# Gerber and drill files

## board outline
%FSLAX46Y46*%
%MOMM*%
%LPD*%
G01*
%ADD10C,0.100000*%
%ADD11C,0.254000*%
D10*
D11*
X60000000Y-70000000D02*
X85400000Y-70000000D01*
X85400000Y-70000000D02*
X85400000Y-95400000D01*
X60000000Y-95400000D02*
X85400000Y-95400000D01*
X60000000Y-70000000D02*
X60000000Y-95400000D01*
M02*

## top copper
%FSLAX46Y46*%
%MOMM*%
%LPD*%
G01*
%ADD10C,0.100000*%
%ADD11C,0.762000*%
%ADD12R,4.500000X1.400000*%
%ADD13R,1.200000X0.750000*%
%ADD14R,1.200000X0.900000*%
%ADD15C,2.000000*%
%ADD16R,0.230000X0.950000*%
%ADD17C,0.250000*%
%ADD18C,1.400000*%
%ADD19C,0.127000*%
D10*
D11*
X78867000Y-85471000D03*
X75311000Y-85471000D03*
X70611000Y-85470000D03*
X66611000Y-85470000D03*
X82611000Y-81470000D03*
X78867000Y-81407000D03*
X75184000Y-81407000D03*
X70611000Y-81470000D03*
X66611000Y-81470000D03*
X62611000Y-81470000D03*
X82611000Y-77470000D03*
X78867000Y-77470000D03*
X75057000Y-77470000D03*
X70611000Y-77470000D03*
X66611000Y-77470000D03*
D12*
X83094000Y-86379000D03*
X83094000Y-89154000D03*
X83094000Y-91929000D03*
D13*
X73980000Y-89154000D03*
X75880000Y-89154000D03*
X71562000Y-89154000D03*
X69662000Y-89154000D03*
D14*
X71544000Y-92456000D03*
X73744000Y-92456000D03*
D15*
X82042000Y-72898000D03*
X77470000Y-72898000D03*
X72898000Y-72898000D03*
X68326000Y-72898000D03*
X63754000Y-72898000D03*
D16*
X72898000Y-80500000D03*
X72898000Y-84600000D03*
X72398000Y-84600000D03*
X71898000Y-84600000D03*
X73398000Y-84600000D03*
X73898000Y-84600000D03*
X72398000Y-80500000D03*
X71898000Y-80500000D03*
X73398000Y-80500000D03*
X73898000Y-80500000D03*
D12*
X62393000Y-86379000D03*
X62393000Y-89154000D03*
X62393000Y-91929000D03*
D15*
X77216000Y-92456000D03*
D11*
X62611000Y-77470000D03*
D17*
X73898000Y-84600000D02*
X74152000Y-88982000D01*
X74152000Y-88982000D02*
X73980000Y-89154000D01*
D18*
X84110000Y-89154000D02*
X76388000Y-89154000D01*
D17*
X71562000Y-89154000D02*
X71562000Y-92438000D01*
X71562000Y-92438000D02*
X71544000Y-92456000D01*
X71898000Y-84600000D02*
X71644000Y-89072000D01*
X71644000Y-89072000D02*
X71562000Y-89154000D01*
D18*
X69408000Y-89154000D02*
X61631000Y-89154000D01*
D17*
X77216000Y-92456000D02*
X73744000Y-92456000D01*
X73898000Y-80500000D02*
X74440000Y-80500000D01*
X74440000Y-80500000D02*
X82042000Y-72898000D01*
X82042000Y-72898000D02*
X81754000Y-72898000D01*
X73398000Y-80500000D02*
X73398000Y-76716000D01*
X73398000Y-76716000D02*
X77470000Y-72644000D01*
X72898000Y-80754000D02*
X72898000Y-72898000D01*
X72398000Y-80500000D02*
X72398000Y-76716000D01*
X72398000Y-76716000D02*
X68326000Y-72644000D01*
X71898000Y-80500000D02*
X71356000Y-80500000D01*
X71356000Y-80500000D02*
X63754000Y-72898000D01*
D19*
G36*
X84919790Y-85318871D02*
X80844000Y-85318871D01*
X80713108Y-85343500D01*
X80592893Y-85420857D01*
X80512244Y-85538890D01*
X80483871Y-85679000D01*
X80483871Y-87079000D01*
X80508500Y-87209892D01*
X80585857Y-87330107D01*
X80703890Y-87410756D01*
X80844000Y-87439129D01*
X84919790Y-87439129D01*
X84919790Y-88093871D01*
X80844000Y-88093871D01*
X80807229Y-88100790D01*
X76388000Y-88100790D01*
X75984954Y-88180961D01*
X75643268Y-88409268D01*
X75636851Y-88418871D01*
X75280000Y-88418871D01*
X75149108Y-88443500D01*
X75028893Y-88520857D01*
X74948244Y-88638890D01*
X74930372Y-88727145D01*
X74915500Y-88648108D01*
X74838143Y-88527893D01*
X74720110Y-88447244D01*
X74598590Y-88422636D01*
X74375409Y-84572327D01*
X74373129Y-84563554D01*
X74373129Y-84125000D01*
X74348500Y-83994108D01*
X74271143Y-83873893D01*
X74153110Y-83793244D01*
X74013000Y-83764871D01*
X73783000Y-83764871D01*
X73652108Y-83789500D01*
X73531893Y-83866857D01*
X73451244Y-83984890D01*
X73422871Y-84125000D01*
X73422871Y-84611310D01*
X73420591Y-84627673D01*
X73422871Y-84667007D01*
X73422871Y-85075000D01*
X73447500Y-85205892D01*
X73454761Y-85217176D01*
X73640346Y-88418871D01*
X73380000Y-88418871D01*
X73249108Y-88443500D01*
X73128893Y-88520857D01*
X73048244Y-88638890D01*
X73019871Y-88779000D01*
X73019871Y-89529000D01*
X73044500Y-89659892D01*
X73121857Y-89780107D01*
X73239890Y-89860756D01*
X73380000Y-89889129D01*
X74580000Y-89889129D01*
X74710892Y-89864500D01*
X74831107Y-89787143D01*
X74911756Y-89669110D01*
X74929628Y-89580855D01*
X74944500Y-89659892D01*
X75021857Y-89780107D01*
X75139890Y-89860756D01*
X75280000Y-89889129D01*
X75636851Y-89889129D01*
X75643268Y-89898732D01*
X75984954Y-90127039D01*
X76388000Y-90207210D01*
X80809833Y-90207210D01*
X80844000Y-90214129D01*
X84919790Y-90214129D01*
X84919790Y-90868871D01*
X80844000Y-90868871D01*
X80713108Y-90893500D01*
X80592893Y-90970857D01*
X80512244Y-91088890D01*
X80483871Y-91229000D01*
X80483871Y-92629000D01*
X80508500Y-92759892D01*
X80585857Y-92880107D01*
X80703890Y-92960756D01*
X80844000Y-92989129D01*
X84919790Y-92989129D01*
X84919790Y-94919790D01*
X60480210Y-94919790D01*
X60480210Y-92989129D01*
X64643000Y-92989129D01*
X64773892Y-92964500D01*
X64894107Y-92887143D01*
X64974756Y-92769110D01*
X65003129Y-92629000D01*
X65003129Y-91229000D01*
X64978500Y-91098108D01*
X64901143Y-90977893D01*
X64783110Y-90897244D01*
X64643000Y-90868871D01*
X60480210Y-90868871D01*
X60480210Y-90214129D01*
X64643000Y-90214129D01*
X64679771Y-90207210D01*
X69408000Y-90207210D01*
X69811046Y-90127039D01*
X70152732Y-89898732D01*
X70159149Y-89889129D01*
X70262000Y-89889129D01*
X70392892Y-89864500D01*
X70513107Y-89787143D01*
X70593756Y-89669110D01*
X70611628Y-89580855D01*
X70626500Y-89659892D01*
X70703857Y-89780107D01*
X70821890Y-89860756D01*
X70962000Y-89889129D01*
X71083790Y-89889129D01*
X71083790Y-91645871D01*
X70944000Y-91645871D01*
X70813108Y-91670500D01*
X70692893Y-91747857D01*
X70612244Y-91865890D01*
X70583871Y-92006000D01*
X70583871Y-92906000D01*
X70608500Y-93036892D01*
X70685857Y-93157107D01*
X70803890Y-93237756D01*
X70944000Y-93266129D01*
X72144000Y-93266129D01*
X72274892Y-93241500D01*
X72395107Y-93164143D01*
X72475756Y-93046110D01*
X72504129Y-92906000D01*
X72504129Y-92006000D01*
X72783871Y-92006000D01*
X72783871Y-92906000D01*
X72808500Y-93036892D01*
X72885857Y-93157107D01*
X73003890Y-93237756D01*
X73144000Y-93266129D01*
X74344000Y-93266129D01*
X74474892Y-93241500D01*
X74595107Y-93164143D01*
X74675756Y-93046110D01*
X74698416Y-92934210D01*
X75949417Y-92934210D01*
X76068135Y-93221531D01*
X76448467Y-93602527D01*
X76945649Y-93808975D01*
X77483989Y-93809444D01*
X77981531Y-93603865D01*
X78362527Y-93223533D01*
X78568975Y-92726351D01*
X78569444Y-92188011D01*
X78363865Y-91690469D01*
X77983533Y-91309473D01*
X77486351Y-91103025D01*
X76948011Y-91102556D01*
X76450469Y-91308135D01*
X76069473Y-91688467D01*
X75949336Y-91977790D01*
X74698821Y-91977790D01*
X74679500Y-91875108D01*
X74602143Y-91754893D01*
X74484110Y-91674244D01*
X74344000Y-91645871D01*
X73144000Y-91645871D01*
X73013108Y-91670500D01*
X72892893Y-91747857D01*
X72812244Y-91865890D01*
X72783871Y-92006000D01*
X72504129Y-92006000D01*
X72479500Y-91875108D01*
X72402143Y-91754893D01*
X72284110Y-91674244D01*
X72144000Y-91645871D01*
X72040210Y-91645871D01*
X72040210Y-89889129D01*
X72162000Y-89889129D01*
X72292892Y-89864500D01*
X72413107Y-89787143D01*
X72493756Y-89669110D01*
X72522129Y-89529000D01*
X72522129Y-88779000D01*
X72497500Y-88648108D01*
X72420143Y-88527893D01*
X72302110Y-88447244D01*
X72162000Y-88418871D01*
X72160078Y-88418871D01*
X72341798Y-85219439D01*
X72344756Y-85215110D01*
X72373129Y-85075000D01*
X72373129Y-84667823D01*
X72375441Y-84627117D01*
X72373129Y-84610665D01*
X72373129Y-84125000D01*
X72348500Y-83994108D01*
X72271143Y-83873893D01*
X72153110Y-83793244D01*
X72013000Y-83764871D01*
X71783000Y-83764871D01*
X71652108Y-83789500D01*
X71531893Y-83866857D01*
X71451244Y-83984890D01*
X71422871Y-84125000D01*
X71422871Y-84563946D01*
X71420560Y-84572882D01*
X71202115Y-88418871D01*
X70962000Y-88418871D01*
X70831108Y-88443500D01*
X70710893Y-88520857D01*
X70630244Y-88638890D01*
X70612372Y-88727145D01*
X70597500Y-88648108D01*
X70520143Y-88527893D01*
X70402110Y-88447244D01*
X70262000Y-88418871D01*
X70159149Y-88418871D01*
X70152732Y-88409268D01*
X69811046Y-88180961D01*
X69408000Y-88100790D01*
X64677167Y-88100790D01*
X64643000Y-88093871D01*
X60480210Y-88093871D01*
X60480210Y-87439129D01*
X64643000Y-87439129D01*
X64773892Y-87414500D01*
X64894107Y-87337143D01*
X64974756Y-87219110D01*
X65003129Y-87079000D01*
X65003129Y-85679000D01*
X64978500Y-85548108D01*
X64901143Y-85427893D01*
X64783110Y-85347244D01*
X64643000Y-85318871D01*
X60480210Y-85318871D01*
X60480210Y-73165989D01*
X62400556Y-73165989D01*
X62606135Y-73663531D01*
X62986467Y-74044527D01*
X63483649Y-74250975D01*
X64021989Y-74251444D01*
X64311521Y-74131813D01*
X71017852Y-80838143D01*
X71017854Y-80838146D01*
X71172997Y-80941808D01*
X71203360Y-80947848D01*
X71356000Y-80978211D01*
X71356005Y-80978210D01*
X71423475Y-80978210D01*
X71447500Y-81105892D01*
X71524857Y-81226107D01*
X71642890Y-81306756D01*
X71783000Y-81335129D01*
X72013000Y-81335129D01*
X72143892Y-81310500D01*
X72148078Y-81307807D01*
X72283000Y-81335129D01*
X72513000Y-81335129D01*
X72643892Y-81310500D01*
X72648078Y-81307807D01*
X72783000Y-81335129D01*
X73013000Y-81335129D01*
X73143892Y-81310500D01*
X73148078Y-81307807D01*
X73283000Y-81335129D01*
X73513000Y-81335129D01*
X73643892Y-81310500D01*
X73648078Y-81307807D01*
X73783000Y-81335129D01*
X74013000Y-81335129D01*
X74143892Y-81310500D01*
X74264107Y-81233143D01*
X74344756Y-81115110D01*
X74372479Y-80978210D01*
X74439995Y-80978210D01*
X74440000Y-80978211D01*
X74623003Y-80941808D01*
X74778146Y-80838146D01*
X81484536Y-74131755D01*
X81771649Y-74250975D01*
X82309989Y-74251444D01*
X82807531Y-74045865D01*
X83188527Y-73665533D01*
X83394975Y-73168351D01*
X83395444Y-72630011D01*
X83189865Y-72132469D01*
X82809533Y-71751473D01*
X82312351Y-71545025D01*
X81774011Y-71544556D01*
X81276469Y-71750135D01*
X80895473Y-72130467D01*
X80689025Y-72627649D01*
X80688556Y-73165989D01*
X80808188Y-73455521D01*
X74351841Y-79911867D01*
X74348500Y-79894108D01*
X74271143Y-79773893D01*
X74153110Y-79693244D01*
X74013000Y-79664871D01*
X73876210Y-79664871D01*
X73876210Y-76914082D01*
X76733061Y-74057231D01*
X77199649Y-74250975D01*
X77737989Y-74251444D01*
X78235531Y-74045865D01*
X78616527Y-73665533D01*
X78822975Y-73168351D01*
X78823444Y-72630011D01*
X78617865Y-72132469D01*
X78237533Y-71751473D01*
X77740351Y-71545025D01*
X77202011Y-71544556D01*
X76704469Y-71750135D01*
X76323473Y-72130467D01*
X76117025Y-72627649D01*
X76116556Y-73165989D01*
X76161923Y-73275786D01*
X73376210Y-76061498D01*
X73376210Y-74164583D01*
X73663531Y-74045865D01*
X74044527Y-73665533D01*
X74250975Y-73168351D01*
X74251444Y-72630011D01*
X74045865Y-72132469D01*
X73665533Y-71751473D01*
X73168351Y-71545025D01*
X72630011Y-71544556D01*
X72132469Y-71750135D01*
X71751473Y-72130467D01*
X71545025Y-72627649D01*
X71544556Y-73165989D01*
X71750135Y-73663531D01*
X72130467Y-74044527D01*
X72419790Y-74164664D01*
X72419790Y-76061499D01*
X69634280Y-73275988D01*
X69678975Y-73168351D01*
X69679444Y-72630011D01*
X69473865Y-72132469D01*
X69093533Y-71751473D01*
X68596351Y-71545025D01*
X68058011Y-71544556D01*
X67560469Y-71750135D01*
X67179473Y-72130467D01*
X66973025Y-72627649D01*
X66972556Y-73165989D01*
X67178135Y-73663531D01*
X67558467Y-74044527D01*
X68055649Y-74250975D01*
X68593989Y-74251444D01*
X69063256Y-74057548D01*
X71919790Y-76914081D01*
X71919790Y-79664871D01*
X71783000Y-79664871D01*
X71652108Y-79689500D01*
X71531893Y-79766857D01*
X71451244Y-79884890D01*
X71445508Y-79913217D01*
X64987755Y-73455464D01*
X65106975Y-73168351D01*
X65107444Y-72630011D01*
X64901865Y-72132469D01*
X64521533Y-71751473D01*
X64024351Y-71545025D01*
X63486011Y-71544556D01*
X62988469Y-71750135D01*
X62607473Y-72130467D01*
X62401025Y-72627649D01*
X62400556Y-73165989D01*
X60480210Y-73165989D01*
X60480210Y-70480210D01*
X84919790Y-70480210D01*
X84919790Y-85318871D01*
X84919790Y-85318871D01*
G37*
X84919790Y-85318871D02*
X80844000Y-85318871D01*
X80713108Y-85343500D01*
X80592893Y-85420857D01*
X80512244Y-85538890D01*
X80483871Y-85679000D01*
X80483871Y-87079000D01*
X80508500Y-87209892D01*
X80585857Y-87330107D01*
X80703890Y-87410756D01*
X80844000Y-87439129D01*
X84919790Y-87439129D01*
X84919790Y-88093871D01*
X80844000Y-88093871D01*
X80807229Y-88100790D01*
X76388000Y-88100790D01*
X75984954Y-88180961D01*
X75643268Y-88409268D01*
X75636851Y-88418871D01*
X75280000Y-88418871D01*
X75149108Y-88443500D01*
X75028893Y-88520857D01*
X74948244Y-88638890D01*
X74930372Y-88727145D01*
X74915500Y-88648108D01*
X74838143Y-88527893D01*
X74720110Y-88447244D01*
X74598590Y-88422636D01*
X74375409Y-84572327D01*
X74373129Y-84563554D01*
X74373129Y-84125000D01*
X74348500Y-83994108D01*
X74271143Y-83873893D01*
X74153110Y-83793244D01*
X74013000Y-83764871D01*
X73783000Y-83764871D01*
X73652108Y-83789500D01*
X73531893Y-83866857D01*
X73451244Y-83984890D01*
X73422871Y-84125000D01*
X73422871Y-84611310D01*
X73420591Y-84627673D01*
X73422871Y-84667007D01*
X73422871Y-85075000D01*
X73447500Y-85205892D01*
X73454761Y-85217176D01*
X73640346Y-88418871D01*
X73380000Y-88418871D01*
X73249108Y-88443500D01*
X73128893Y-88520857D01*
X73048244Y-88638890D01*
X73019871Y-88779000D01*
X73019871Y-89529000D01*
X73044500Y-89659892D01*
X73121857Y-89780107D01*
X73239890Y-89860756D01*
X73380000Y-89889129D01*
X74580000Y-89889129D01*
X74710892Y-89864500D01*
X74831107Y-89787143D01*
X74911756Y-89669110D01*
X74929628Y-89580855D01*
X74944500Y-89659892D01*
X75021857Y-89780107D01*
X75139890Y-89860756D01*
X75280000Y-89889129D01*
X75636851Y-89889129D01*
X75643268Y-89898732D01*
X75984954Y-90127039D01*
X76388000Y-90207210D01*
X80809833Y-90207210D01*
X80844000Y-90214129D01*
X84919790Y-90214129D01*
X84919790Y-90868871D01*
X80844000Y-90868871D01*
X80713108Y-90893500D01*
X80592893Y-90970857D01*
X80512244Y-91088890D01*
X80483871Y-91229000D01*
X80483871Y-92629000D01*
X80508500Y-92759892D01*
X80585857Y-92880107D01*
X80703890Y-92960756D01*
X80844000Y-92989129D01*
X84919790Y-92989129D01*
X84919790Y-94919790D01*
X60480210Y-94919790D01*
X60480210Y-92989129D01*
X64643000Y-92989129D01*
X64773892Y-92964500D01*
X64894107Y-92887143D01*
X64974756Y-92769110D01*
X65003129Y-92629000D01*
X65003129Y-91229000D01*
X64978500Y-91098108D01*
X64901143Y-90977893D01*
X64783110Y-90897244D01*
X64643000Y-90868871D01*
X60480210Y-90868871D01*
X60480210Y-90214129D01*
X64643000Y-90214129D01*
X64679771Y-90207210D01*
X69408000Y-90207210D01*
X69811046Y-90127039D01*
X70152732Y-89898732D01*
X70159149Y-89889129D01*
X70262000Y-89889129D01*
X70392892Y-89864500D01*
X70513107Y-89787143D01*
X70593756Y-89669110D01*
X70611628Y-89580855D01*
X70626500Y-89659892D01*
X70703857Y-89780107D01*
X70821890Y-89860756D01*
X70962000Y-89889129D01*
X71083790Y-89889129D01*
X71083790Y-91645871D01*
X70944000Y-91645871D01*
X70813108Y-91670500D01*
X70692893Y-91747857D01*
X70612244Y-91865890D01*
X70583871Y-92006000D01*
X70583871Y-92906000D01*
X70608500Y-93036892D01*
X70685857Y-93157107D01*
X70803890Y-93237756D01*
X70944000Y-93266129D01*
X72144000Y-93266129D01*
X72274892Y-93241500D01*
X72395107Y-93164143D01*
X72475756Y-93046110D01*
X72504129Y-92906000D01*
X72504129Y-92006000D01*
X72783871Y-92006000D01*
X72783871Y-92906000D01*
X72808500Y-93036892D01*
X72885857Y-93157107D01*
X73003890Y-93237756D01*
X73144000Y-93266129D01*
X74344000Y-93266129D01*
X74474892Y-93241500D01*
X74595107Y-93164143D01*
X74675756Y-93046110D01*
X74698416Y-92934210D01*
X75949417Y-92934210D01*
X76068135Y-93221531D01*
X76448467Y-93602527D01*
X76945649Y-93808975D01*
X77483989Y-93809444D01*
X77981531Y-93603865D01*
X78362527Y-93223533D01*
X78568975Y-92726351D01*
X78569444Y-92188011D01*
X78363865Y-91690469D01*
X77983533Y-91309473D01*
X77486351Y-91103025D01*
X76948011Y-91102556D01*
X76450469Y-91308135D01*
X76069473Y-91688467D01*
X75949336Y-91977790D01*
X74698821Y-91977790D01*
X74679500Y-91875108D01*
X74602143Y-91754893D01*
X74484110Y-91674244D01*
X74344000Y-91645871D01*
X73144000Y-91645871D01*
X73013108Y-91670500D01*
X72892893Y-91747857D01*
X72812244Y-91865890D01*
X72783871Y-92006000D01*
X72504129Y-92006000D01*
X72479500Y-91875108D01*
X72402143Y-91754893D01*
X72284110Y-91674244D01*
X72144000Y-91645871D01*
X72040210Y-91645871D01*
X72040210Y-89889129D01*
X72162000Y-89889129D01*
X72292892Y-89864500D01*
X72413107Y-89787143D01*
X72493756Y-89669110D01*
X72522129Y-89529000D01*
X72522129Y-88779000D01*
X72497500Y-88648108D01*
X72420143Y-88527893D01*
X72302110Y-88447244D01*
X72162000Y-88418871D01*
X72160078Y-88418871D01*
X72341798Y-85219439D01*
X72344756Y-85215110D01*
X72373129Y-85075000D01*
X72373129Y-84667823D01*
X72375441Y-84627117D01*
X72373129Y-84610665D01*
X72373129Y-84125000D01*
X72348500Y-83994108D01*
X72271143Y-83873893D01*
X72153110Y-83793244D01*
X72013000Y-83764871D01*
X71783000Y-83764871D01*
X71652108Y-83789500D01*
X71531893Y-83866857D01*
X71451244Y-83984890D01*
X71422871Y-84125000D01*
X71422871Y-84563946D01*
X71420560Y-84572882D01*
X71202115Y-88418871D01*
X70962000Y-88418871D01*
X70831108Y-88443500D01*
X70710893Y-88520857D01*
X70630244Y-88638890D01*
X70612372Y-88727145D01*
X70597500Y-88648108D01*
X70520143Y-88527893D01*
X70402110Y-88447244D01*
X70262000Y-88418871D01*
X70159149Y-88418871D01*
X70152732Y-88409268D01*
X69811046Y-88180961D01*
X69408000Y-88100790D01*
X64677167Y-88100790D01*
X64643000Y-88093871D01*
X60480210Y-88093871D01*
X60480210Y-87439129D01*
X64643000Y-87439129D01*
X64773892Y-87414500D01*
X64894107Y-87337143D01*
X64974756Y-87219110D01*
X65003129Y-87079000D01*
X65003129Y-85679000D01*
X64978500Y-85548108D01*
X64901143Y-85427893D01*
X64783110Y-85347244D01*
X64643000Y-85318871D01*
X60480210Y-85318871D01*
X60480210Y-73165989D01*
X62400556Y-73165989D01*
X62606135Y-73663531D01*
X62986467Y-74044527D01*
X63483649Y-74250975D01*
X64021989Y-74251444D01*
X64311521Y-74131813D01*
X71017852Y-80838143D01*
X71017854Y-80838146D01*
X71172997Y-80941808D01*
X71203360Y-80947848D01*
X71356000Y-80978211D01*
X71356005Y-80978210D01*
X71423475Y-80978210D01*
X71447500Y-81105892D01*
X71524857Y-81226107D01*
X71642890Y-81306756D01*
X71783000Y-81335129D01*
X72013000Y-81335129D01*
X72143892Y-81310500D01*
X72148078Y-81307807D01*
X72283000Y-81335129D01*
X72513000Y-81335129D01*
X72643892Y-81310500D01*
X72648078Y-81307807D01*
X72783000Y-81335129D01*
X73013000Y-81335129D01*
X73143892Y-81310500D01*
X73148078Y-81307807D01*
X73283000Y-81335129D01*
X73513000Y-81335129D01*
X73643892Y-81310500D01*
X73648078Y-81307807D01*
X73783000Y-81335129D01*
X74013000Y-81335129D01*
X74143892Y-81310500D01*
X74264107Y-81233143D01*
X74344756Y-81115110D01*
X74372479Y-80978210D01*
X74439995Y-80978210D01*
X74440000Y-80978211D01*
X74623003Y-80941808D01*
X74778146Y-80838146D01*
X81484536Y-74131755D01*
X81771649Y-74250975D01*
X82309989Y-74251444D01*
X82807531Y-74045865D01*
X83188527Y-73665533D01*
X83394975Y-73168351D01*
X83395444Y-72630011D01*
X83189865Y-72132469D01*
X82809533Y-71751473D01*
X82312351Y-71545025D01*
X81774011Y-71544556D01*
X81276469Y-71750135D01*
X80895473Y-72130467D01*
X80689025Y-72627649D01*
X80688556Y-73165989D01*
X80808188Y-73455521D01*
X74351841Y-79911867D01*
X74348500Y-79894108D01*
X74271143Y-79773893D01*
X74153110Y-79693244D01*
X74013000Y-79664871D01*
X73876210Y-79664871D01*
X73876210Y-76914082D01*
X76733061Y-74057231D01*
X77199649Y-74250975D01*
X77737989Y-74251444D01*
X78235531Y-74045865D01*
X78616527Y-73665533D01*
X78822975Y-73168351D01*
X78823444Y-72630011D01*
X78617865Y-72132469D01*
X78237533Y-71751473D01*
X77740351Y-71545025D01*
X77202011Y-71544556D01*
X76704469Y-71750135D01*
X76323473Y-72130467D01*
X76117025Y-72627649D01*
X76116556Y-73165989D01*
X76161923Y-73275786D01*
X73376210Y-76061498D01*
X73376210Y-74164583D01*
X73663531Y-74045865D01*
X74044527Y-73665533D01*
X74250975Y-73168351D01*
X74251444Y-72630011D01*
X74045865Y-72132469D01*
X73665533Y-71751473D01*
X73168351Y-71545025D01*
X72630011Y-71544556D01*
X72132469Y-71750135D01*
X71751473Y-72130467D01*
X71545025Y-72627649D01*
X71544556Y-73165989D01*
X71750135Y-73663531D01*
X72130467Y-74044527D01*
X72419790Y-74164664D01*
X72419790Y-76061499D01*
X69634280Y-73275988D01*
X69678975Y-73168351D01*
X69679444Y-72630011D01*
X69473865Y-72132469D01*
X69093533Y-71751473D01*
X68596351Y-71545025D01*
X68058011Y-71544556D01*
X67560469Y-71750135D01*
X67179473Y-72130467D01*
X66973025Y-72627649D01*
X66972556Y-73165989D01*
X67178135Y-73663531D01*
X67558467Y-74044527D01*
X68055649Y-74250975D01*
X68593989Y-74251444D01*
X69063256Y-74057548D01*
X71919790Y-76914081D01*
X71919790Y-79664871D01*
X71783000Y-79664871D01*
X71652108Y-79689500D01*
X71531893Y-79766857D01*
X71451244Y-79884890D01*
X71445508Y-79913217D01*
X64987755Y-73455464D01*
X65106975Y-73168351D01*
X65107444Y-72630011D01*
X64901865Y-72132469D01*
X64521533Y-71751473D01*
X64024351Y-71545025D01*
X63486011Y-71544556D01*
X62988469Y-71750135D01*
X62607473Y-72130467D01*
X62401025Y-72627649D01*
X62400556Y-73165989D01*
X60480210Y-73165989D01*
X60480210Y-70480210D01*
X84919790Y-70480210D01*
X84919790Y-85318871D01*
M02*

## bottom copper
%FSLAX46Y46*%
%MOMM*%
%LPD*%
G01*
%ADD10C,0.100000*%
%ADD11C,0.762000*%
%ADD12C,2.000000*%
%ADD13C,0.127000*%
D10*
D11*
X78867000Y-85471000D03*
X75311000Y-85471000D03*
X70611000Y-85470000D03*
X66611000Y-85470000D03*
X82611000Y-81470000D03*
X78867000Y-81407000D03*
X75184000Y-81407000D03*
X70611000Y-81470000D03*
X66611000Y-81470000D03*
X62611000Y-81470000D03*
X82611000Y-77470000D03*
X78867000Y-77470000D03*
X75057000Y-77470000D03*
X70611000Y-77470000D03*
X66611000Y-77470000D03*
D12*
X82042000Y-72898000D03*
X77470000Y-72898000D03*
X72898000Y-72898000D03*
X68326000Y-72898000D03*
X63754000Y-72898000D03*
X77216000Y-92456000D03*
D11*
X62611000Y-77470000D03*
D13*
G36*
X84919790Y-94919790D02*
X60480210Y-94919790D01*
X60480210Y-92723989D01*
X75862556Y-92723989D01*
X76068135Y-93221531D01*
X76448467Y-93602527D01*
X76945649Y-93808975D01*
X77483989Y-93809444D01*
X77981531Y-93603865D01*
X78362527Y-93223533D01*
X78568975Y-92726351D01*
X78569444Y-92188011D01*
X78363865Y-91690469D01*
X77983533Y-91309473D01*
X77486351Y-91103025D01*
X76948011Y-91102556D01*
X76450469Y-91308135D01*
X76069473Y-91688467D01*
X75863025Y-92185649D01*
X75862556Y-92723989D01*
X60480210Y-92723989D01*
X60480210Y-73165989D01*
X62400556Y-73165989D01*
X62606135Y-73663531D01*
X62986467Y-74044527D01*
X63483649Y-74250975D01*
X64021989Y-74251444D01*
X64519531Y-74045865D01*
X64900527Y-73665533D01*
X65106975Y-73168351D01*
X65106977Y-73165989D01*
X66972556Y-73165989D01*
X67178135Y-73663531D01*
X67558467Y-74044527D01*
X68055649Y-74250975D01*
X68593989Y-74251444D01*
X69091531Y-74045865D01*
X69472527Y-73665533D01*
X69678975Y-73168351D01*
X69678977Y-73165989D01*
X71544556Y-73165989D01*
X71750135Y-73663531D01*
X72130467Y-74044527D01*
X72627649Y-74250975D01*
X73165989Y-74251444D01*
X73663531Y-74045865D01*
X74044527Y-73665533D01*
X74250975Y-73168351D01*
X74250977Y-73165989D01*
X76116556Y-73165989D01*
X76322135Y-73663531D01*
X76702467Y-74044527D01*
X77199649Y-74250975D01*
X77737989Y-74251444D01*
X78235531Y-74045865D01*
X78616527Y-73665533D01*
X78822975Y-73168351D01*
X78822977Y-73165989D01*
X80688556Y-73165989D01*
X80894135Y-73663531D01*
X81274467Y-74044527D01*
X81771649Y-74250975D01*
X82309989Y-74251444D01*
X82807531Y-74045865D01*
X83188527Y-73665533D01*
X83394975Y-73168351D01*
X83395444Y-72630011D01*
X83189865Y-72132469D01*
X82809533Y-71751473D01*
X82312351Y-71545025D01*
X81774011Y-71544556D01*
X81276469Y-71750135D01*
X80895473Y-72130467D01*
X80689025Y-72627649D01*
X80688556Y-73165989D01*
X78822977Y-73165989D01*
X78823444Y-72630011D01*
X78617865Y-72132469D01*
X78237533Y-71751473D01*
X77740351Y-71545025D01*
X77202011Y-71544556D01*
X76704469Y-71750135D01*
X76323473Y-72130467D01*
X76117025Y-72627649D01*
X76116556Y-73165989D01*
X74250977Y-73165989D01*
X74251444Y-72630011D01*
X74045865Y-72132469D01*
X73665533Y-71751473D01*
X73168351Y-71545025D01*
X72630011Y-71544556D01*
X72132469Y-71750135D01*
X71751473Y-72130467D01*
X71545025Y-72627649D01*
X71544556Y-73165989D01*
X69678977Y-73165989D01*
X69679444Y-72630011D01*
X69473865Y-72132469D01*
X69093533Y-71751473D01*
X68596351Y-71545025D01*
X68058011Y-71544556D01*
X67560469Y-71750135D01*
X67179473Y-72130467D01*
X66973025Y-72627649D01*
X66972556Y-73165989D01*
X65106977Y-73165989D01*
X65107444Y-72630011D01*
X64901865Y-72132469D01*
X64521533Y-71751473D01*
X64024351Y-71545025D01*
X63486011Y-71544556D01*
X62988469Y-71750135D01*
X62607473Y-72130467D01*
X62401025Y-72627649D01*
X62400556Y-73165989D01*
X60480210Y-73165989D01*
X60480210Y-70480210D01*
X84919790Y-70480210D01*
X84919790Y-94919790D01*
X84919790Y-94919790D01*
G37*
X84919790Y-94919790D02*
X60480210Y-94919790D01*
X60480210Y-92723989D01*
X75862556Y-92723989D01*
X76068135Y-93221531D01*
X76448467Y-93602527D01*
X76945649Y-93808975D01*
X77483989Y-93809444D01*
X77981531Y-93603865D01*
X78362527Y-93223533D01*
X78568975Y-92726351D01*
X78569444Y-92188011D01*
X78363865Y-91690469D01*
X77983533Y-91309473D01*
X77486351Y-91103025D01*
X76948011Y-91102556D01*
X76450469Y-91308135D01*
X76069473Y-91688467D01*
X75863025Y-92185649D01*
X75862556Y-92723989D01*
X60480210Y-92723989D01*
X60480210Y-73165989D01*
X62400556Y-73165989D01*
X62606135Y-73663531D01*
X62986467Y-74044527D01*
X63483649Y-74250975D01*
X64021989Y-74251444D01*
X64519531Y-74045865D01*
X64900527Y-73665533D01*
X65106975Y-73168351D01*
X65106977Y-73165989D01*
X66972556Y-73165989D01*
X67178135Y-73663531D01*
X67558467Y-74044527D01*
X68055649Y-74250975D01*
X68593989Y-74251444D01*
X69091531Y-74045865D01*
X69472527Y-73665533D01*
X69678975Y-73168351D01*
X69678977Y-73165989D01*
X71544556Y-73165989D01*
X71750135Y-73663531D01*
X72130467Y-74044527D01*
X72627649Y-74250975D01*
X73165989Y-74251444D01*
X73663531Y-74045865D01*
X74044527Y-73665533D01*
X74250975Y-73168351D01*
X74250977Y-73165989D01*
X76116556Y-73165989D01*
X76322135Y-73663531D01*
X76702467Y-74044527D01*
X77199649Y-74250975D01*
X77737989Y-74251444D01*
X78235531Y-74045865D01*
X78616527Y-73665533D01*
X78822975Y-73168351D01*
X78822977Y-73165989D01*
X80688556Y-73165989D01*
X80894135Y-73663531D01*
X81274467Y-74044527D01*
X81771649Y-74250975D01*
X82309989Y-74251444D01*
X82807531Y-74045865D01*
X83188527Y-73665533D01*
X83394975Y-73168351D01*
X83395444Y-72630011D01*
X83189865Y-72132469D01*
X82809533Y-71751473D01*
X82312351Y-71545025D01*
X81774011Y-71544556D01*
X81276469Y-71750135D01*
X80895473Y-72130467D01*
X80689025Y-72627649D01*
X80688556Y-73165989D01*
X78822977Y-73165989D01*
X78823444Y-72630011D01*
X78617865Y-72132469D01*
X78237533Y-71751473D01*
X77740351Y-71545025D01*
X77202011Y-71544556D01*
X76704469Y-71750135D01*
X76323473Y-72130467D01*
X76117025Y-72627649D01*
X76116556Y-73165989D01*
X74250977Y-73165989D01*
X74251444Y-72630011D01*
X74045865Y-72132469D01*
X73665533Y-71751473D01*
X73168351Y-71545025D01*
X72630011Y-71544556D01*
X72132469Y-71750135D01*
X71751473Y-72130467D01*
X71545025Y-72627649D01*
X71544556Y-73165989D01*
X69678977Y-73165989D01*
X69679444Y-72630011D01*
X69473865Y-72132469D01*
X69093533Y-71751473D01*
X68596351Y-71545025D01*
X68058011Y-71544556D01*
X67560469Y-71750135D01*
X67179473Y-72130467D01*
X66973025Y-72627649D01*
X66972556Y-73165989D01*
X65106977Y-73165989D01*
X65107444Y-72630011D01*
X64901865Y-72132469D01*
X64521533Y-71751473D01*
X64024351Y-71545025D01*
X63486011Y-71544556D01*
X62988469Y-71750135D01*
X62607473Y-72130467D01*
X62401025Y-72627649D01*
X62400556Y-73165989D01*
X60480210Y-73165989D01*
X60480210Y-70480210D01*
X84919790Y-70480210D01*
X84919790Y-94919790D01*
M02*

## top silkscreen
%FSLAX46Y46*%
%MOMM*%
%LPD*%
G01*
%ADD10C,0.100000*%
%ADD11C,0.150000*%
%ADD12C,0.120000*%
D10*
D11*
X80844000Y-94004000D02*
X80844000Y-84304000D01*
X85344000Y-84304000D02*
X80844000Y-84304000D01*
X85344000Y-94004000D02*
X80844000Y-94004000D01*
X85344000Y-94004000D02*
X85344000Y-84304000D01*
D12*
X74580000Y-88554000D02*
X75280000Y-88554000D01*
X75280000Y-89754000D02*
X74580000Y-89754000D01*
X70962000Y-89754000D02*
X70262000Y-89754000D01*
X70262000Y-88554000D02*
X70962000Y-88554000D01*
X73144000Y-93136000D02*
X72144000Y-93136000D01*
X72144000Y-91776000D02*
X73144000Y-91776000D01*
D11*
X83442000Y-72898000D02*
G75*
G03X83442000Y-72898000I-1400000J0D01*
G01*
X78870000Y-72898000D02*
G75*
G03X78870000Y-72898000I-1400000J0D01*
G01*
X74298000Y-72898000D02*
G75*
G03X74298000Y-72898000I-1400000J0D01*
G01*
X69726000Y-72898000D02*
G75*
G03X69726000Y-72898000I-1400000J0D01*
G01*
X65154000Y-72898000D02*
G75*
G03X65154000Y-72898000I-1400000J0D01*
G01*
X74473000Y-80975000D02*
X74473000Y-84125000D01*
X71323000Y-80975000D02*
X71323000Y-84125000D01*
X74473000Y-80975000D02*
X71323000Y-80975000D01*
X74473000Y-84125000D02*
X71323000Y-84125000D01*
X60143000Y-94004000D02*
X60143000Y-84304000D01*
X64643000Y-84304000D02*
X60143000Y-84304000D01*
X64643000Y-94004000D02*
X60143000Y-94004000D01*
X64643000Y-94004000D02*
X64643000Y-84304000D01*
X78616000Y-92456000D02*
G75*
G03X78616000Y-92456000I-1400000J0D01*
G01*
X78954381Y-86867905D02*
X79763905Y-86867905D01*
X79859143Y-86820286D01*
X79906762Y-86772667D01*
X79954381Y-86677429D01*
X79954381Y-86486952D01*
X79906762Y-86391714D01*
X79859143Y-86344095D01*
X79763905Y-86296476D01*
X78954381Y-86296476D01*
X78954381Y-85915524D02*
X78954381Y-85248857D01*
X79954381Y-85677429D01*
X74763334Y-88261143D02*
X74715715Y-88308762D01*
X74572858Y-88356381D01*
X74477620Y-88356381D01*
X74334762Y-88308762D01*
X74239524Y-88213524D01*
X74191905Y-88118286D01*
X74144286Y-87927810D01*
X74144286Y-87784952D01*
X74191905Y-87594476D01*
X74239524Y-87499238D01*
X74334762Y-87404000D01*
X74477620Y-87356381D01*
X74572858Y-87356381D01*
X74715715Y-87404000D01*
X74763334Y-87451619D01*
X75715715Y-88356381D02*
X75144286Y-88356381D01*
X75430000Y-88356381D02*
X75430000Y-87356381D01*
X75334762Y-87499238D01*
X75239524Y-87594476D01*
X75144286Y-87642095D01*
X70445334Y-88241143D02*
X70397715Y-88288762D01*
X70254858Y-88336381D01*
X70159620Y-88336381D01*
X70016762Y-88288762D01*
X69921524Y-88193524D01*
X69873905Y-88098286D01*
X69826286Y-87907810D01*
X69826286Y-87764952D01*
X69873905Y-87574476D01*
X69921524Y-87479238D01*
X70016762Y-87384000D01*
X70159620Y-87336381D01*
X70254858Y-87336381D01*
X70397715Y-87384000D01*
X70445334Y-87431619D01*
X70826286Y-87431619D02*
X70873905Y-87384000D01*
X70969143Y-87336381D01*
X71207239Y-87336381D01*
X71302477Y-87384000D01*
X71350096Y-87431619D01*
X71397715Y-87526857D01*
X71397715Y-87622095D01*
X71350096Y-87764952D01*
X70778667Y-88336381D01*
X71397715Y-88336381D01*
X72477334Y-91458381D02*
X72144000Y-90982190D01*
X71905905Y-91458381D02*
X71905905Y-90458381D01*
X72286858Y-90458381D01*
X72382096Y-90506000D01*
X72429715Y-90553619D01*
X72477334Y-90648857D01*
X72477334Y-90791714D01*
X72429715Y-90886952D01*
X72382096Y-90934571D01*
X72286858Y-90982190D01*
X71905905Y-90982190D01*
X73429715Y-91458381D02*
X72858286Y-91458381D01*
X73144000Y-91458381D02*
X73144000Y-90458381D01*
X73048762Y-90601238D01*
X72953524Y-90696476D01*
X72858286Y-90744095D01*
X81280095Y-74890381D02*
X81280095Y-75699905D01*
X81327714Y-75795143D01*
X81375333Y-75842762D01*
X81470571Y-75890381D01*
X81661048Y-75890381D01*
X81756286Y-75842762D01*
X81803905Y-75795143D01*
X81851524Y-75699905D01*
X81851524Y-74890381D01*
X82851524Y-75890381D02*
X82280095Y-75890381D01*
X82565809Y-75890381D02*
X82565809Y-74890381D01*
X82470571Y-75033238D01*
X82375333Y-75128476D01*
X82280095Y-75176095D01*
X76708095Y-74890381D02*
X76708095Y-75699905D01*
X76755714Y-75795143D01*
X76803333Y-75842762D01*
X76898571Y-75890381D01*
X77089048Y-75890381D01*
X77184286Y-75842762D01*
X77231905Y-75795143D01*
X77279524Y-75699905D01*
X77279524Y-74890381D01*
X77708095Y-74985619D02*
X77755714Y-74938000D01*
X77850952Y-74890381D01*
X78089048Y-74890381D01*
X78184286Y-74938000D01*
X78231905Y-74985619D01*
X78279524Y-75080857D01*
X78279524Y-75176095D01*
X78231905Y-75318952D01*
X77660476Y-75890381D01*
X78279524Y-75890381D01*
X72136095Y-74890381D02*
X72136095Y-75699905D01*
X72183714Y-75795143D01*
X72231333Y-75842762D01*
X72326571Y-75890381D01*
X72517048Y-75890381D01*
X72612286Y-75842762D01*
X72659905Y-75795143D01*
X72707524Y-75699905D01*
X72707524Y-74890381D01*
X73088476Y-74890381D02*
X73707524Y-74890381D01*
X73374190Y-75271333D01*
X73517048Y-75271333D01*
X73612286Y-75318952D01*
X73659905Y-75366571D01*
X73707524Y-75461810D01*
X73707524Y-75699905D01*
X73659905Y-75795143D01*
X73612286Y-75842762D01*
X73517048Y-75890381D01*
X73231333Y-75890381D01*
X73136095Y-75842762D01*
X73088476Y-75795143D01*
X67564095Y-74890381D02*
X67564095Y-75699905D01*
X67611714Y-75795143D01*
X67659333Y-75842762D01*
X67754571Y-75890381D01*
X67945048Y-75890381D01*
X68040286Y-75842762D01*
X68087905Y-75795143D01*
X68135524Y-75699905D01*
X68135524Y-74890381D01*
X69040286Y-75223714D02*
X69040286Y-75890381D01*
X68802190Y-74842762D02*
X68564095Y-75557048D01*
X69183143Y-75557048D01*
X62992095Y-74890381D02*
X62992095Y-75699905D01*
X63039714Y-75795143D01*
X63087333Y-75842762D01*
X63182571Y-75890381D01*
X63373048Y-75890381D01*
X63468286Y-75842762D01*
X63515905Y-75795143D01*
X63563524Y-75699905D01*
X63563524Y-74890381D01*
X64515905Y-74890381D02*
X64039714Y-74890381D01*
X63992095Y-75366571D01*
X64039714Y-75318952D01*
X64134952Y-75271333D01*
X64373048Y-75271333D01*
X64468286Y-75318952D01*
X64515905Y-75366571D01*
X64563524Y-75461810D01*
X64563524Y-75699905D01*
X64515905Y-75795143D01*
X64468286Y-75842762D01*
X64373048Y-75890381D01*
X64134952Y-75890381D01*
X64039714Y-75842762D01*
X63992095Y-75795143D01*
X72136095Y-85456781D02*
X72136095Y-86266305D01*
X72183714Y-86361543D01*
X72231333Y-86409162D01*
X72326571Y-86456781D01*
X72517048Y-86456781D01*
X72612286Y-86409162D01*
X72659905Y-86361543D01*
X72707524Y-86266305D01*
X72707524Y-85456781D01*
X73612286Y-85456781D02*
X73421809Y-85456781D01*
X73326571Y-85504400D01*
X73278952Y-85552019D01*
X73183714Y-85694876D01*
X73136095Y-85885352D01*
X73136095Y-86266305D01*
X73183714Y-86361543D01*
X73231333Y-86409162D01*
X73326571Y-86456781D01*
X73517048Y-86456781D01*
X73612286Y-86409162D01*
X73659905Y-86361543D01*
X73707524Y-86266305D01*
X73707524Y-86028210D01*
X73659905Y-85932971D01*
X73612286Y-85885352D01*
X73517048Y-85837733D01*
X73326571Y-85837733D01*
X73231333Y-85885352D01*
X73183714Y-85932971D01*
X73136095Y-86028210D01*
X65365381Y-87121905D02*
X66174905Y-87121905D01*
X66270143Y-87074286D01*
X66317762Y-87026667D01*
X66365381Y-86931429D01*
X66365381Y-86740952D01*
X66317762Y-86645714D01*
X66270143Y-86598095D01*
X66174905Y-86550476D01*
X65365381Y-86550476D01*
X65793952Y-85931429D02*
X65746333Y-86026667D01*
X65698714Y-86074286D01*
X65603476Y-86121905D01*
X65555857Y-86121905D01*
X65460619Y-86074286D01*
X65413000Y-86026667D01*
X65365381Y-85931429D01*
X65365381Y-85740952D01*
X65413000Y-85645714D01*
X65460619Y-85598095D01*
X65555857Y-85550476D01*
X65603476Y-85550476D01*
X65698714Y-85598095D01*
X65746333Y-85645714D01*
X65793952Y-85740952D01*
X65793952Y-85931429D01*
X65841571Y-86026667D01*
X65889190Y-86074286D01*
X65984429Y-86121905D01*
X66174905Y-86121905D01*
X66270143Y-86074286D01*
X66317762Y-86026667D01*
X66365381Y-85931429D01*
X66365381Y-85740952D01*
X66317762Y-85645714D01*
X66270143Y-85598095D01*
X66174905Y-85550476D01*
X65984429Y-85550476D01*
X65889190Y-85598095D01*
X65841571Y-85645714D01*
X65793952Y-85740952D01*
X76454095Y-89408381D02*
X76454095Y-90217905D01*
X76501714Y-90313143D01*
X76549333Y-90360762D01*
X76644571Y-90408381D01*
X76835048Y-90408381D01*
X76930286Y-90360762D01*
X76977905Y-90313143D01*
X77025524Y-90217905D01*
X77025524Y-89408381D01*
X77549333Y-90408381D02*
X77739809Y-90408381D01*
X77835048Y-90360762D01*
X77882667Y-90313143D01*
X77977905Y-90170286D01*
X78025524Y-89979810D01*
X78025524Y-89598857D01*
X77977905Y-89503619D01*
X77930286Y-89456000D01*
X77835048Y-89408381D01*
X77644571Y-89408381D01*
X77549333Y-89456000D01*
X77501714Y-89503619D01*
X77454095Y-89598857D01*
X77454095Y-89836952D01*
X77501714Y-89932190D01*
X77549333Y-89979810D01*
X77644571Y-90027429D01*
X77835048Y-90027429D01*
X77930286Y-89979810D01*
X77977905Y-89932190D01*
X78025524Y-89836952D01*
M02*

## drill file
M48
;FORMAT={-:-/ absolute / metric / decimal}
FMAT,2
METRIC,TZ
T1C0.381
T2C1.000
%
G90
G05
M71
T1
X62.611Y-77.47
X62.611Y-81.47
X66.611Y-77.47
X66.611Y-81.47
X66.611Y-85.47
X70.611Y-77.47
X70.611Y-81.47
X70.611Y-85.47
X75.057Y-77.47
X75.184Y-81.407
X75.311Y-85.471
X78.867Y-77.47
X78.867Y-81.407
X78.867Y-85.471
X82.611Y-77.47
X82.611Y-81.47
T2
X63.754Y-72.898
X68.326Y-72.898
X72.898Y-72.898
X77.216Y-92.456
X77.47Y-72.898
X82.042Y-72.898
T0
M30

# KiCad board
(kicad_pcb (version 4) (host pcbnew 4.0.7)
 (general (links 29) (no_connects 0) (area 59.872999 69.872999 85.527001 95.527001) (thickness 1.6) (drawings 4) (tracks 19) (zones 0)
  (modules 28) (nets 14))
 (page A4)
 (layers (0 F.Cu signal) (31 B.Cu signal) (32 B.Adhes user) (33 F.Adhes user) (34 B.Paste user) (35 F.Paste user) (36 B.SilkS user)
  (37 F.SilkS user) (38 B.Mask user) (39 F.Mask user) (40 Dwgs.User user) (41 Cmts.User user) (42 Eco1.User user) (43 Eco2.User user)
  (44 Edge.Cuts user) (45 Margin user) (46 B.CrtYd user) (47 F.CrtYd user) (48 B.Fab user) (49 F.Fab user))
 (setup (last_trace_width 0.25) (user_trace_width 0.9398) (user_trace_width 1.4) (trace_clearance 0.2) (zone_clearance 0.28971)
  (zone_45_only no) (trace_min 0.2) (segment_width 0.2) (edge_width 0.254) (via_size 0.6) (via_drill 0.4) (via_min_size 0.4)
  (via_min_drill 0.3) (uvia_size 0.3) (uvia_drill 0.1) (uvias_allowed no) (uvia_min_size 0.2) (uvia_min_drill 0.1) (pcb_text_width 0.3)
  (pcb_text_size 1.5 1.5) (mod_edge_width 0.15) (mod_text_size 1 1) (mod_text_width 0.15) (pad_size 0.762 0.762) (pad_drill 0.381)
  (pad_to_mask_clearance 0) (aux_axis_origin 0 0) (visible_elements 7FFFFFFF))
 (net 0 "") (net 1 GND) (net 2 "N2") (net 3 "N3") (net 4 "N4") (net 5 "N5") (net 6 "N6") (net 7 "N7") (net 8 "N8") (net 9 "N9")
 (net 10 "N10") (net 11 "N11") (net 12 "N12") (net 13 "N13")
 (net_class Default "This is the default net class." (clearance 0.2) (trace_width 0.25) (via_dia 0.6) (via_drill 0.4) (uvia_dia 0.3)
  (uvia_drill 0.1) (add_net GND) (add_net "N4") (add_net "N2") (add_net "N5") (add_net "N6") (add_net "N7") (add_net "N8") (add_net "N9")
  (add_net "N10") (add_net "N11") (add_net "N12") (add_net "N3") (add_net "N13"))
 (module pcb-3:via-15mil (layer B.Cu) (at 78.867 85.471)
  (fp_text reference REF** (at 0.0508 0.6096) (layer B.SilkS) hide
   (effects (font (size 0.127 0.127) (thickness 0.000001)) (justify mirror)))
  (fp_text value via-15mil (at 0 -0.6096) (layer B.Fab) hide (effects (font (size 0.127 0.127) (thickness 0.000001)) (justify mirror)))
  (pad 1 thru_hole circle (at 0 0) (size 0.762 0.762) (drill 0.381) (layers *.Cu) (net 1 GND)))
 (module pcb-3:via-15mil (layer F.Cu) (at 75.311 85.471)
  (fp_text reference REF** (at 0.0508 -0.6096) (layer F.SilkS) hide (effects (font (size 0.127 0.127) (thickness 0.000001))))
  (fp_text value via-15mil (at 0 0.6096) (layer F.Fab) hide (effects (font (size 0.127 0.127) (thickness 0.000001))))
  (pad 1 thru_hole circle (at 0 0) (size 0.762 0.762) (drill 0.381) (layers *.Cu) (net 1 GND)))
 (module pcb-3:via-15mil (layer F.Cu) (at 70.611 85.47)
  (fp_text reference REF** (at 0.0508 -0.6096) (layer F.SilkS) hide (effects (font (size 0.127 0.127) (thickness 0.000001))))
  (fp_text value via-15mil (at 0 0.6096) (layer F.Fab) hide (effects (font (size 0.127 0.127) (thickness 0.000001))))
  (pad 1 thru_hole circle (at 0 0) (size 0.762 0.762) (drill 0.381) (layers *.Cu) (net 1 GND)))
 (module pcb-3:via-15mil (layer F.Cu) (at 66.611 85.47)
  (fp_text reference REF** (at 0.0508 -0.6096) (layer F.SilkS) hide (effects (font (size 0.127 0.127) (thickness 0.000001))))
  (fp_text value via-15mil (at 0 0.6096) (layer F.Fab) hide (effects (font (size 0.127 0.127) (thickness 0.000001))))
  (pad 1 thru_hole circle (at 0 0) (size 0.762 0.762) (drill 0.381) (layers *.Cu) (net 1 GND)))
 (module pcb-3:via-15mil (layer F.Cu) (at 82.611 81.47)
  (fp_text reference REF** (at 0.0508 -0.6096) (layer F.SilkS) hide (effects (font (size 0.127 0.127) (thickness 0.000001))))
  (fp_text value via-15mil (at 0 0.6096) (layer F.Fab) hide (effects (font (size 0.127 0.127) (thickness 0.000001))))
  (pad 1 thru_hole circle (at 0 0) (size 0.762 0.762) (drill 0.381) (layers *.Cu) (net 1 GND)))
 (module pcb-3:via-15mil (layer F.Cu) (at 78.867 81.407)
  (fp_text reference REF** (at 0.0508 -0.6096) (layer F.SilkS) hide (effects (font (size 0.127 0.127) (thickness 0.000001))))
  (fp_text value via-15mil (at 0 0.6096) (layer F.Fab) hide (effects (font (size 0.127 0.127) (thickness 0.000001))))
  (pad 1 thru_hole circle (at 0 0) (size 0.762 0.762) (drill 0.381) (layers *.Cu) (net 1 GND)))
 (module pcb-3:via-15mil (layer F.Cu) (at 75.184 81.407)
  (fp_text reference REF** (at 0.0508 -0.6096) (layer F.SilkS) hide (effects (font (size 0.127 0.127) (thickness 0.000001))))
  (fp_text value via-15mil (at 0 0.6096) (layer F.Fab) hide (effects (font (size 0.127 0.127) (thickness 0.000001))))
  (pad 1 thru_hole circle (at 0 0) (size 0.762 0.762) (drill 0.381) (layers *.Cu) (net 1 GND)))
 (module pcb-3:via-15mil (layer F.Cu) (at 70.611 81.47)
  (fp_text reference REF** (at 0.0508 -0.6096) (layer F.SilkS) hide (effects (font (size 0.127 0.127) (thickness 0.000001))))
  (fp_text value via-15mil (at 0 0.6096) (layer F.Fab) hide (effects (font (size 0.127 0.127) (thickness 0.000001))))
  (pad 1 thru_hole circle (at 0 0) (size 0.762 0.762) (drill 0.381) (layers *.Cu) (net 1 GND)))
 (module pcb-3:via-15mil (layer F.Cu) (at 66.611 81.47)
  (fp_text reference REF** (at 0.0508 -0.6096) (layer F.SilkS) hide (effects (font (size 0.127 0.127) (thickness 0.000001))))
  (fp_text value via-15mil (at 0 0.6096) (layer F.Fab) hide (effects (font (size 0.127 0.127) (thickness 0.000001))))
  (pad 1 thru_hole circle (at 0 0) (size 0.762 0.762) (drill 0.381) (layers *.Cu) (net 1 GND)))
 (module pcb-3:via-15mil (layer F.Cu) (at 62.611 81.47)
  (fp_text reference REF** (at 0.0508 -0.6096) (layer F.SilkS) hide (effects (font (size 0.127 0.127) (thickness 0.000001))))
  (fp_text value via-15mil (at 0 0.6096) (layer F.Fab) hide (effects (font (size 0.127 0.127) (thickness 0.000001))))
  (pad 1 thru_hole circle (at 0 0) (size 0.762 0.762) (drill 0.381) (layers *.Cu) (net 1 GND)))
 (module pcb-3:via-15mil (layer F.Cu) (at 82.611 77.47)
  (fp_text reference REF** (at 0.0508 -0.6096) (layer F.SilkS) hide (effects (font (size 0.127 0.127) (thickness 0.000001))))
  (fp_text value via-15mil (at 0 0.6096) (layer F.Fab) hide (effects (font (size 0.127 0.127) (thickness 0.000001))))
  (pad 1 thru_hole circle (at 0 0) (size 0.762 0.762) (drill 0.381) (layers *.Cu) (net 1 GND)))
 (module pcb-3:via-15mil (layer F.Cu) (at 78.867 77.47)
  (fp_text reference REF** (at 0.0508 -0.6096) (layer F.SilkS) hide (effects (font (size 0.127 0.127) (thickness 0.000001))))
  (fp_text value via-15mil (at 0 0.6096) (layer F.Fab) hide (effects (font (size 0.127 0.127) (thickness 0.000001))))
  (pad 1 thru_hole circle (at 0 0) (size 0.762 0.762) (drill 0.381) (layers *.Cu) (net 1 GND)))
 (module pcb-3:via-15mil (layer F.Cu) (at 75.057 77.47)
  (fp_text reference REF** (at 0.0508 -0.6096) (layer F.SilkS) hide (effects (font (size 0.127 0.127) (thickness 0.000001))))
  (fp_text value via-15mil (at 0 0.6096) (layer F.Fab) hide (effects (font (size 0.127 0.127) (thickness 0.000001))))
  (pad 1 thru_hole circle (at 0 0) (size 0.762 0.762) (drill 0.381) (layers *.Cu) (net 1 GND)))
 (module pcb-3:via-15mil (layer F.Cu) (at 70.611 77.47)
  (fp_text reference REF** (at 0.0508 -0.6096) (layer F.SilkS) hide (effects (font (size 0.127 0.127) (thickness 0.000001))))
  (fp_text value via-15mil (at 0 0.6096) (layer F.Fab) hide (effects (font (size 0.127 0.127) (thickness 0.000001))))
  (pad 1 thru_hole circle (at 0 0) (size 0.762 0.762) (drill 0.381) (layers *.Cu) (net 1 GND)))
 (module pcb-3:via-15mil (layer F.Cu) (at 66.611 77.47)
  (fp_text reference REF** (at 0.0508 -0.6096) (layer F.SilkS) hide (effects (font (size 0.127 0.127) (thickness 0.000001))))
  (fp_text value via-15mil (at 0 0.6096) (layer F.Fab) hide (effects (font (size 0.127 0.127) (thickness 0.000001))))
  (pad 1 thru_hole circle (at 0 0) (size 0.762 0.762) (drill 0.381) (layers *.Cu) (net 1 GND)))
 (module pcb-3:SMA (layer F.Cu) (at 85.344 89.154 90)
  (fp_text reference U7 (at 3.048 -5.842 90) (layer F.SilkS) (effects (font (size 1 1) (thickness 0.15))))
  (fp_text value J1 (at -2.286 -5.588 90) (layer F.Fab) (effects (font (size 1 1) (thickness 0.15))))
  (fp_line (start -4.85 -4.5) (end 4.85 -4.5) (layer F.SilkS) (width 0.15))
  (fp_line (start 4.85 0) (end 4.85 -4.5) (layer F.SilkS) (width 0.15))
  (fp_line (start -4.85 0) (end -4.85 -4.5) (layer F.SilkS) (width 0.15))
  (fp_line (start -4.85 0) (end 4.85 0) (layer F.SilkS) (width 0.15))
  (pad 3 connect rect (at 2.775 -2.25 90) (size 1.4 4.5) (layers F.Cu F.Mask))
  (pad 2 connect rect (at 0 -2.25 90) (size 1.4 4.5) (layers F.Cu F.Mask) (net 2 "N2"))
  (pad 1 connect rect (at -2.775 -2.25 90) (size 1.4 4.5) (layers F.Cu F.Mask) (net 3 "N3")))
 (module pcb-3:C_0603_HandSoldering (layer F.Cu) (at 74.93 89.154)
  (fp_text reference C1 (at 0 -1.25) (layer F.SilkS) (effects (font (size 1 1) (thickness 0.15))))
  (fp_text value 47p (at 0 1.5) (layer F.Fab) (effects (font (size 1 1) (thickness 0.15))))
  (fp_line (start -0.35 -0.6) (end 0.35 -0.6) (layer F.SilkS) (width 0.12))
  (fp_line (start 0.35 0.6) (end -0.35 0.6) (layer F.SilkS) (width 0.12))
  (pad 1 smd rect (at -0.95 0) (size 1.2 0.75) (layers F.Cu F.Paste F.Mask) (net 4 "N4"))
  (pad 2 smd rect (at 0.95 0) (size 1.2 0.75) (layers F.Cu F.Paste F.Mask) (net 2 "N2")))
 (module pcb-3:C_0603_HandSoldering (layer F.Cu) (at 70.612 89.154 180)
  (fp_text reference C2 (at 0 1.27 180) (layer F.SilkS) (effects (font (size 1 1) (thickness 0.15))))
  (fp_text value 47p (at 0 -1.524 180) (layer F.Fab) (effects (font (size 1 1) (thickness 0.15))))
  (fp_line (start -0.35 -0.6) (end 0.35 -0.6) (layer F.SilkS) (width 0.12))
  (fp_line (start 0.35 0.6) (end -0.35 0.6) (layer F.SilkS) (width 0.12))
  (pad 1 smd rect (at -0.95 0 180) (size 1.2 0.75) (layers F.Cu F.Paste F.Mask) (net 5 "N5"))
  (pad 2 smd rect (at 0.95 0 180) (size 1.2 0.75) (layers F.Cu F.Paste F.Mask) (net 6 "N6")))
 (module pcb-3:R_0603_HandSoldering (layer F.Cu) (at 72.644 92.456)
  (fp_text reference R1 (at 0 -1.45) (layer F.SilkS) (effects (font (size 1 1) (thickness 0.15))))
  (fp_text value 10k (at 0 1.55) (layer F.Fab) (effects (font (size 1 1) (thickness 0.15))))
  (fp_line (start 0.5 0.68) (end -0.5 0.68) (layer F.SilkS) (width 0.12))
  (fp_line (start -0.5 -0.68) (end 0.5 -0.68) (layer F.SilkS) (width 0.12))
  (pad 1 smd rect (at -1.1 0) (size 1.2 0.9) (layers F.Cu F.Paste F.Mask) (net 5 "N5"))
  (pad 2 smd rect (at 1.1 0) (size 1.2 0.9) (layers F.Cu F.Paste F.Mask) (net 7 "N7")))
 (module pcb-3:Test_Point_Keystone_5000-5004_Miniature (layer F.Cu) (at 82.042 72.898)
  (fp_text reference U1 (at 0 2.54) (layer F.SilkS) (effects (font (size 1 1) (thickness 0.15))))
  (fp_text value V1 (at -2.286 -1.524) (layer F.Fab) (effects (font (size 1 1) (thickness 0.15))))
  (fp_circle (center 0 0) (end 1.4 0) (layer F.SilkS) (width 0.15))
  (pad 1 thru_hole circle (at 0 0) (size 2 2) (drill 1) (layers *.Cu *.Mask) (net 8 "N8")))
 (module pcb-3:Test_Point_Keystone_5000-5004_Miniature (layer F.Cu) (at 77.47 72.898)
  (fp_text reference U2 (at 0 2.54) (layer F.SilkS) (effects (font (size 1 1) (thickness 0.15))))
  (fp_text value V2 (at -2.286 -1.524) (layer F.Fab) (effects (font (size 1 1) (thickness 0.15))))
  (fp_circle (center 0 0) (end 1.4 0) (layer F.SilkS) (width 0.15))
  (pad 1 thru_hole circle (at 0 0) (size 2 2) (drill 1) (layers *.Cu *.Mask) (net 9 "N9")))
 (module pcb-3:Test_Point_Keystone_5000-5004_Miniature (layer F.Cu) (at 72.898 72.898)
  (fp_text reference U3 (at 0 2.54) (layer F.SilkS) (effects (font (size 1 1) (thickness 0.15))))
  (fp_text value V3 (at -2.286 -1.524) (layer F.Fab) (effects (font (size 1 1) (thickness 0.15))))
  (fp_circle (center 0 0) (end 1.4 0) (layer F.SilkS) (width 0.15))
  (pad 1 thru_hole circle (at 0 0) (size 2 2) (drill 1) (layers *.Cu *.Mask) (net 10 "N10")))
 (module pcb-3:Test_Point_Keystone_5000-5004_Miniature (layer F.Cu) (at 68.326 72.898)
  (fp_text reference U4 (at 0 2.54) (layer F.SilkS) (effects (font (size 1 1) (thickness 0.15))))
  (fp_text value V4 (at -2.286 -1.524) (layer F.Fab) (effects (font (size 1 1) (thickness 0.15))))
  (fp_circle (center 0 0) (end 1.4 0) (layer F.SilkS) (width 0.15))
  (pad 1 thru_hole circle (at 0 0) (size 2 2) (drill 1) (layers *.Cu *.Mask) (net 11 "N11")))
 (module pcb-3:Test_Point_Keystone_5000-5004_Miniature (layer F.Cu) (at 63.754 72.898)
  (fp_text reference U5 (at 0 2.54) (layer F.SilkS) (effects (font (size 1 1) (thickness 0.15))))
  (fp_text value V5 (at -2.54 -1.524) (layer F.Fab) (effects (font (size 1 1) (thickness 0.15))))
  (fp_circle (center 0 0) (end 1.4 0) (layer F.SilkS) (width 0.15))
  (pad 1 thru_hole circle (at 0 0) (size 2 2) (drill 1) (layers *.Cu *.Mask) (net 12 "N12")))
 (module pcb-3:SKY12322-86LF (layer F.Cu) (at 72.898 82.55 180)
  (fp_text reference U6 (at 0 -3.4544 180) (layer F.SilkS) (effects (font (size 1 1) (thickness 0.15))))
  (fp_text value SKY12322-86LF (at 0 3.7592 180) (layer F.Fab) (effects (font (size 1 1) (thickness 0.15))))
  (fp_line (start -1.575 1.575) (end -1.575 -1.575) (layer F.SilkS) (width 0.15))
  (fp_line (start 1.575 1.575) (end 1.575 -1.575) (layer F.SilkS) (width 0.15))
  (fp_line (start -1.575 1.575) (end 1.575 1.575) (layer F.SilkS) (width 0.15))
  (fp_line (start -1.575 -1.575) (end 1.575 -1.575) (layer F.SilkS) (width 0.15))
  (pad 3 smd rect (at 0 2.05 180) (size 0.23 0.95) (layers F.Cu F.Paste F.Mask) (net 10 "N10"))
  (pad 8 smd rect (at 0 -2.05 180) (size 0.23 0.95) (layers F.Cu F.Paste F.Mask) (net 1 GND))
  (pad 7 smd rect (at 0.5 -2.05 180) (size 0.23 0.95) (layers F.Cu F.Paste F.Mask) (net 1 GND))
  (pad 6 smd rect (at 1 -2.05 180) (size 0.23 0.95) (layers F.Cu F.Paste F.Mask) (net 5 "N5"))
  (pad 9 smd rect (at -0.5 -2.05 180) (size 0.23 0.95) (layers F.Cu F.Paste F.Mask) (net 1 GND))
  (pad 10 smd rect (at -1 -2.05 180) (size 0.23 0.95) (layers F.Cu F.Paste F.Mask) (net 4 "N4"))
  (pad 4 smd rect (at 0.5 2.05 180) (size 0.23 0.95) (layers F.Cu F.Paste F.Mask) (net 11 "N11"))
  (pad 5 smd rect (at 1 2.05 180) (size 0.23 0.95) (layers F.Cu F.Paste F.Mask) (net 12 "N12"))
  (pad 2 smd rect (at -0.5 2.05 180) (size 0.23 0.95) (layers F.Cu F.Paste F.Mask) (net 9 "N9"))
  (pad 1 smd rect (at -1 2.05 180) (size 0.23 0.95) (layers F.Cu F.Paste F.Mask) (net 8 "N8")))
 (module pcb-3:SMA (layer F.Cu) (at 64.643 89.154 90)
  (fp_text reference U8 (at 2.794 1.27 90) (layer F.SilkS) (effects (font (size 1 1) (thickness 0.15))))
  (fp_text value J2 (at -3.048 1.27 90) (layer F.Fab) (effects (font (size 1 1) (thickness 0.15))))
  (fp_line (start -4.85 -4.5) (end 4.85 -4.5) (layer F.SilkS) (width 0.15))
  (fp_line (start 4.85 0) (end 4.85 -4.5) (layer F.SilkS) (width 0.15))
  (fp_line (start -4.85 0) (end -4.85 -4.5) (layer F.SilkS) (width 0.15))
  (fp_line (start -4.85 0) (end 4.85 0) (layer F.SilkS) (width 0.15))
  (pad 3 connect rect (at 2.775 -2.25 90) (size 1.4 4.5) (layers F.Cu F.Mask))
  (pad 2 connect rect (at 0 -2.25 90) (size 1.4 4.5) (layers F.Cu F.Mask) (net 6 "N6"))
  (pad 1 connect rect (at -2.775 -2.25 90) (size 1.4 4.5) (layers F.Cu F.Mask) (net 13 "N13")))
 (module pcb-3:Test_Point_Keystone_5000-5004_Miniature (layer F.Cu) (at 77.216 92.456)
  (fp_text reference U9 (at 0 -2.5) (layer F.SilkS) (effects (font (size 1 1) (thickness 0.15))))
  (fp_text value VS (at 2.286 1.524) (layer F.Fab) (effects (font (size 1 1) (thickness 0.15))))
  (fp_circle (center 0 0) (end 1.4 0) (layer F.SilkS) (width 0.15))
  (pad 1 thru_hole circle (at 0 0) (size 2 2) (drill 1) (layers *.Cu *.Mask) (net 7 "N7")))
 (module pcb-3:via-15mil (layer F.Cu) (at 62.611 77.47)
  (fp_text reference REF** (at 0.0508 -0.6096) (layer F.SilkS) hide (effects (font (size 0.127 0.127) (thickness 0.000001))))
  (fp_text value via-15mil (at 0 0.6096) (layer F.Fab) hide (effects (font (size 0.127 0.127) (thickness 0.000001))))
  (pad 1 thru_hole circle (at 0 0) (size 0.762 0.762) (drill 0.381) (layers *.Cu) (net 1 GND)))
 (gr_line (start 60 70) (end 85.4 70) (angle 90) (layer Edge.Cuts) (width 0.254))
 (gr_line (start 85.4 70) (end 85.4 95.4) (angle 90) (layer Edge.Cuts) (width 0.254))
 (gr_line (start 60 95.4) (end 85.4 95.4) (angle 90) (layer Edge.Cuts) (width 0.254))
 (gr_line (start 60 70) (end 60 95.4) (angle 90) (layer Edge.Cuts) (width 0.254))
 (segment (start 73.898 84.6) (end 74.152 88.982) (width 0.25) (layer F.Cu) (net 4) (status 20))
 (segment (start 74.152 88.982) (end 73.98 89.154) (width 0.25) (layer F.Cu) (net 4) (status 30))
 (segment (start 84.11 89.154) (end 76.388 89.154) (width 1.4) (layer F.Cu) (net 2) (status 10))
 (segment (start 71.562 89.154) (end 71.562 92.438) (width 0.25) (layer F.Cu) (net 5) (status 20))
 (segment (start 71.562 92.438) (end 71.544 92.456) (width 0.25) (layer F.Cu) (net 5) (status 30))
 (segment (start 71.898 84.6) (end 71.644 89.072) (width 0.25) (layer F.Cu) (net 5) (status 20))
 (segment (start 71.644 89.072) (end 71.562 89.154) (width 0.25) (layer F.Cu) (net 5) (status 30))
 (segment (start 69.408 89.154) (end 61.631 89.154) (width 1.4) (layer F.Cu) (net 6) (status 20))
 (segment (start 77.216 92.456) (end 73.744 92.456) (width 0.25) (layer F.Cu) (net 7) (status 10))
 (segment (start 73.898 80.5) (end 74.44 80.5) (width 0.25) (layer F.Cu) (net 8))
 (segment (start 74.44 80.5) (end 82.042 72.898) (width 0.25) (layer F.Cu) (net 8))
 (segment (start 82.042 72.898) (end 81.754 72.898) (width 0.25) (layer F.Cu) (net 8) (status 30))
 (segment (start 73.398 80.5) (end 73.398 76.716) (width 0.25) (layer F.Cu) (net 9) (status 10))
 (segment (start 73.398 76.716) (end 77.47 72.644) (width 0.25) (layer F.Cu) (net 9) (status 20))
 (segment (start 72.898 80.754) (end 72.898 72.898) (width 0.25) (layer F.Cu) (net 10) (status 20))
 (segment (start 72.398 80.5) (end 72.398 76.716) (width 0.25) (layer F.Cu) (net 11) (status 10))
 (segment (start 72.398 76.716) (end 68.326 72.644) (width 0.25) (layer F.Cu) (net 11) (status 20))
 (segment (start 71.898 80.5) (end 71.356 80.5) (width 0.25) (layer F.Cu) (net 12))
 (segment (start 71.356 80.5) (end 63.754 72.898) (width 0.25) (layer F.Cu) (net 12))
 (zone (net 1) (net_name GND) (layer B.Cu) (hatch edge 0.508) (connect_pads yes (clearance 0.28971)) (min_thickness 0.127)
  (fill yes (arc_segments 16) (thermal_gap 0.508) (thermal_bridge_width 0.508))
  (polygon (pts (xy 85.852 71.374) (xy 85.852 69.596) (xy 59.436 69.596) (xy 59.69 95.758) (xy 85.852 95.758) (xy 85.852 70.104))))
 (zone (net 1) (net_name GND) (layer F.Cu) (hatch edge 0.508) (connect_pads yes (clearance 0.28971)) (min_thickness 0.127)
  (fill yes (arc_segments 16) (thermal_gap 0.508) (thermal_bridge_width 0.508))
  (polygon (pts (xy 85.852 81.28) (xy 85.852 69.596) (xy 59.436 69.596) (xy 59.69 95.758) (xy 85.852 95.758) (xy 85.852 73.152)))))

